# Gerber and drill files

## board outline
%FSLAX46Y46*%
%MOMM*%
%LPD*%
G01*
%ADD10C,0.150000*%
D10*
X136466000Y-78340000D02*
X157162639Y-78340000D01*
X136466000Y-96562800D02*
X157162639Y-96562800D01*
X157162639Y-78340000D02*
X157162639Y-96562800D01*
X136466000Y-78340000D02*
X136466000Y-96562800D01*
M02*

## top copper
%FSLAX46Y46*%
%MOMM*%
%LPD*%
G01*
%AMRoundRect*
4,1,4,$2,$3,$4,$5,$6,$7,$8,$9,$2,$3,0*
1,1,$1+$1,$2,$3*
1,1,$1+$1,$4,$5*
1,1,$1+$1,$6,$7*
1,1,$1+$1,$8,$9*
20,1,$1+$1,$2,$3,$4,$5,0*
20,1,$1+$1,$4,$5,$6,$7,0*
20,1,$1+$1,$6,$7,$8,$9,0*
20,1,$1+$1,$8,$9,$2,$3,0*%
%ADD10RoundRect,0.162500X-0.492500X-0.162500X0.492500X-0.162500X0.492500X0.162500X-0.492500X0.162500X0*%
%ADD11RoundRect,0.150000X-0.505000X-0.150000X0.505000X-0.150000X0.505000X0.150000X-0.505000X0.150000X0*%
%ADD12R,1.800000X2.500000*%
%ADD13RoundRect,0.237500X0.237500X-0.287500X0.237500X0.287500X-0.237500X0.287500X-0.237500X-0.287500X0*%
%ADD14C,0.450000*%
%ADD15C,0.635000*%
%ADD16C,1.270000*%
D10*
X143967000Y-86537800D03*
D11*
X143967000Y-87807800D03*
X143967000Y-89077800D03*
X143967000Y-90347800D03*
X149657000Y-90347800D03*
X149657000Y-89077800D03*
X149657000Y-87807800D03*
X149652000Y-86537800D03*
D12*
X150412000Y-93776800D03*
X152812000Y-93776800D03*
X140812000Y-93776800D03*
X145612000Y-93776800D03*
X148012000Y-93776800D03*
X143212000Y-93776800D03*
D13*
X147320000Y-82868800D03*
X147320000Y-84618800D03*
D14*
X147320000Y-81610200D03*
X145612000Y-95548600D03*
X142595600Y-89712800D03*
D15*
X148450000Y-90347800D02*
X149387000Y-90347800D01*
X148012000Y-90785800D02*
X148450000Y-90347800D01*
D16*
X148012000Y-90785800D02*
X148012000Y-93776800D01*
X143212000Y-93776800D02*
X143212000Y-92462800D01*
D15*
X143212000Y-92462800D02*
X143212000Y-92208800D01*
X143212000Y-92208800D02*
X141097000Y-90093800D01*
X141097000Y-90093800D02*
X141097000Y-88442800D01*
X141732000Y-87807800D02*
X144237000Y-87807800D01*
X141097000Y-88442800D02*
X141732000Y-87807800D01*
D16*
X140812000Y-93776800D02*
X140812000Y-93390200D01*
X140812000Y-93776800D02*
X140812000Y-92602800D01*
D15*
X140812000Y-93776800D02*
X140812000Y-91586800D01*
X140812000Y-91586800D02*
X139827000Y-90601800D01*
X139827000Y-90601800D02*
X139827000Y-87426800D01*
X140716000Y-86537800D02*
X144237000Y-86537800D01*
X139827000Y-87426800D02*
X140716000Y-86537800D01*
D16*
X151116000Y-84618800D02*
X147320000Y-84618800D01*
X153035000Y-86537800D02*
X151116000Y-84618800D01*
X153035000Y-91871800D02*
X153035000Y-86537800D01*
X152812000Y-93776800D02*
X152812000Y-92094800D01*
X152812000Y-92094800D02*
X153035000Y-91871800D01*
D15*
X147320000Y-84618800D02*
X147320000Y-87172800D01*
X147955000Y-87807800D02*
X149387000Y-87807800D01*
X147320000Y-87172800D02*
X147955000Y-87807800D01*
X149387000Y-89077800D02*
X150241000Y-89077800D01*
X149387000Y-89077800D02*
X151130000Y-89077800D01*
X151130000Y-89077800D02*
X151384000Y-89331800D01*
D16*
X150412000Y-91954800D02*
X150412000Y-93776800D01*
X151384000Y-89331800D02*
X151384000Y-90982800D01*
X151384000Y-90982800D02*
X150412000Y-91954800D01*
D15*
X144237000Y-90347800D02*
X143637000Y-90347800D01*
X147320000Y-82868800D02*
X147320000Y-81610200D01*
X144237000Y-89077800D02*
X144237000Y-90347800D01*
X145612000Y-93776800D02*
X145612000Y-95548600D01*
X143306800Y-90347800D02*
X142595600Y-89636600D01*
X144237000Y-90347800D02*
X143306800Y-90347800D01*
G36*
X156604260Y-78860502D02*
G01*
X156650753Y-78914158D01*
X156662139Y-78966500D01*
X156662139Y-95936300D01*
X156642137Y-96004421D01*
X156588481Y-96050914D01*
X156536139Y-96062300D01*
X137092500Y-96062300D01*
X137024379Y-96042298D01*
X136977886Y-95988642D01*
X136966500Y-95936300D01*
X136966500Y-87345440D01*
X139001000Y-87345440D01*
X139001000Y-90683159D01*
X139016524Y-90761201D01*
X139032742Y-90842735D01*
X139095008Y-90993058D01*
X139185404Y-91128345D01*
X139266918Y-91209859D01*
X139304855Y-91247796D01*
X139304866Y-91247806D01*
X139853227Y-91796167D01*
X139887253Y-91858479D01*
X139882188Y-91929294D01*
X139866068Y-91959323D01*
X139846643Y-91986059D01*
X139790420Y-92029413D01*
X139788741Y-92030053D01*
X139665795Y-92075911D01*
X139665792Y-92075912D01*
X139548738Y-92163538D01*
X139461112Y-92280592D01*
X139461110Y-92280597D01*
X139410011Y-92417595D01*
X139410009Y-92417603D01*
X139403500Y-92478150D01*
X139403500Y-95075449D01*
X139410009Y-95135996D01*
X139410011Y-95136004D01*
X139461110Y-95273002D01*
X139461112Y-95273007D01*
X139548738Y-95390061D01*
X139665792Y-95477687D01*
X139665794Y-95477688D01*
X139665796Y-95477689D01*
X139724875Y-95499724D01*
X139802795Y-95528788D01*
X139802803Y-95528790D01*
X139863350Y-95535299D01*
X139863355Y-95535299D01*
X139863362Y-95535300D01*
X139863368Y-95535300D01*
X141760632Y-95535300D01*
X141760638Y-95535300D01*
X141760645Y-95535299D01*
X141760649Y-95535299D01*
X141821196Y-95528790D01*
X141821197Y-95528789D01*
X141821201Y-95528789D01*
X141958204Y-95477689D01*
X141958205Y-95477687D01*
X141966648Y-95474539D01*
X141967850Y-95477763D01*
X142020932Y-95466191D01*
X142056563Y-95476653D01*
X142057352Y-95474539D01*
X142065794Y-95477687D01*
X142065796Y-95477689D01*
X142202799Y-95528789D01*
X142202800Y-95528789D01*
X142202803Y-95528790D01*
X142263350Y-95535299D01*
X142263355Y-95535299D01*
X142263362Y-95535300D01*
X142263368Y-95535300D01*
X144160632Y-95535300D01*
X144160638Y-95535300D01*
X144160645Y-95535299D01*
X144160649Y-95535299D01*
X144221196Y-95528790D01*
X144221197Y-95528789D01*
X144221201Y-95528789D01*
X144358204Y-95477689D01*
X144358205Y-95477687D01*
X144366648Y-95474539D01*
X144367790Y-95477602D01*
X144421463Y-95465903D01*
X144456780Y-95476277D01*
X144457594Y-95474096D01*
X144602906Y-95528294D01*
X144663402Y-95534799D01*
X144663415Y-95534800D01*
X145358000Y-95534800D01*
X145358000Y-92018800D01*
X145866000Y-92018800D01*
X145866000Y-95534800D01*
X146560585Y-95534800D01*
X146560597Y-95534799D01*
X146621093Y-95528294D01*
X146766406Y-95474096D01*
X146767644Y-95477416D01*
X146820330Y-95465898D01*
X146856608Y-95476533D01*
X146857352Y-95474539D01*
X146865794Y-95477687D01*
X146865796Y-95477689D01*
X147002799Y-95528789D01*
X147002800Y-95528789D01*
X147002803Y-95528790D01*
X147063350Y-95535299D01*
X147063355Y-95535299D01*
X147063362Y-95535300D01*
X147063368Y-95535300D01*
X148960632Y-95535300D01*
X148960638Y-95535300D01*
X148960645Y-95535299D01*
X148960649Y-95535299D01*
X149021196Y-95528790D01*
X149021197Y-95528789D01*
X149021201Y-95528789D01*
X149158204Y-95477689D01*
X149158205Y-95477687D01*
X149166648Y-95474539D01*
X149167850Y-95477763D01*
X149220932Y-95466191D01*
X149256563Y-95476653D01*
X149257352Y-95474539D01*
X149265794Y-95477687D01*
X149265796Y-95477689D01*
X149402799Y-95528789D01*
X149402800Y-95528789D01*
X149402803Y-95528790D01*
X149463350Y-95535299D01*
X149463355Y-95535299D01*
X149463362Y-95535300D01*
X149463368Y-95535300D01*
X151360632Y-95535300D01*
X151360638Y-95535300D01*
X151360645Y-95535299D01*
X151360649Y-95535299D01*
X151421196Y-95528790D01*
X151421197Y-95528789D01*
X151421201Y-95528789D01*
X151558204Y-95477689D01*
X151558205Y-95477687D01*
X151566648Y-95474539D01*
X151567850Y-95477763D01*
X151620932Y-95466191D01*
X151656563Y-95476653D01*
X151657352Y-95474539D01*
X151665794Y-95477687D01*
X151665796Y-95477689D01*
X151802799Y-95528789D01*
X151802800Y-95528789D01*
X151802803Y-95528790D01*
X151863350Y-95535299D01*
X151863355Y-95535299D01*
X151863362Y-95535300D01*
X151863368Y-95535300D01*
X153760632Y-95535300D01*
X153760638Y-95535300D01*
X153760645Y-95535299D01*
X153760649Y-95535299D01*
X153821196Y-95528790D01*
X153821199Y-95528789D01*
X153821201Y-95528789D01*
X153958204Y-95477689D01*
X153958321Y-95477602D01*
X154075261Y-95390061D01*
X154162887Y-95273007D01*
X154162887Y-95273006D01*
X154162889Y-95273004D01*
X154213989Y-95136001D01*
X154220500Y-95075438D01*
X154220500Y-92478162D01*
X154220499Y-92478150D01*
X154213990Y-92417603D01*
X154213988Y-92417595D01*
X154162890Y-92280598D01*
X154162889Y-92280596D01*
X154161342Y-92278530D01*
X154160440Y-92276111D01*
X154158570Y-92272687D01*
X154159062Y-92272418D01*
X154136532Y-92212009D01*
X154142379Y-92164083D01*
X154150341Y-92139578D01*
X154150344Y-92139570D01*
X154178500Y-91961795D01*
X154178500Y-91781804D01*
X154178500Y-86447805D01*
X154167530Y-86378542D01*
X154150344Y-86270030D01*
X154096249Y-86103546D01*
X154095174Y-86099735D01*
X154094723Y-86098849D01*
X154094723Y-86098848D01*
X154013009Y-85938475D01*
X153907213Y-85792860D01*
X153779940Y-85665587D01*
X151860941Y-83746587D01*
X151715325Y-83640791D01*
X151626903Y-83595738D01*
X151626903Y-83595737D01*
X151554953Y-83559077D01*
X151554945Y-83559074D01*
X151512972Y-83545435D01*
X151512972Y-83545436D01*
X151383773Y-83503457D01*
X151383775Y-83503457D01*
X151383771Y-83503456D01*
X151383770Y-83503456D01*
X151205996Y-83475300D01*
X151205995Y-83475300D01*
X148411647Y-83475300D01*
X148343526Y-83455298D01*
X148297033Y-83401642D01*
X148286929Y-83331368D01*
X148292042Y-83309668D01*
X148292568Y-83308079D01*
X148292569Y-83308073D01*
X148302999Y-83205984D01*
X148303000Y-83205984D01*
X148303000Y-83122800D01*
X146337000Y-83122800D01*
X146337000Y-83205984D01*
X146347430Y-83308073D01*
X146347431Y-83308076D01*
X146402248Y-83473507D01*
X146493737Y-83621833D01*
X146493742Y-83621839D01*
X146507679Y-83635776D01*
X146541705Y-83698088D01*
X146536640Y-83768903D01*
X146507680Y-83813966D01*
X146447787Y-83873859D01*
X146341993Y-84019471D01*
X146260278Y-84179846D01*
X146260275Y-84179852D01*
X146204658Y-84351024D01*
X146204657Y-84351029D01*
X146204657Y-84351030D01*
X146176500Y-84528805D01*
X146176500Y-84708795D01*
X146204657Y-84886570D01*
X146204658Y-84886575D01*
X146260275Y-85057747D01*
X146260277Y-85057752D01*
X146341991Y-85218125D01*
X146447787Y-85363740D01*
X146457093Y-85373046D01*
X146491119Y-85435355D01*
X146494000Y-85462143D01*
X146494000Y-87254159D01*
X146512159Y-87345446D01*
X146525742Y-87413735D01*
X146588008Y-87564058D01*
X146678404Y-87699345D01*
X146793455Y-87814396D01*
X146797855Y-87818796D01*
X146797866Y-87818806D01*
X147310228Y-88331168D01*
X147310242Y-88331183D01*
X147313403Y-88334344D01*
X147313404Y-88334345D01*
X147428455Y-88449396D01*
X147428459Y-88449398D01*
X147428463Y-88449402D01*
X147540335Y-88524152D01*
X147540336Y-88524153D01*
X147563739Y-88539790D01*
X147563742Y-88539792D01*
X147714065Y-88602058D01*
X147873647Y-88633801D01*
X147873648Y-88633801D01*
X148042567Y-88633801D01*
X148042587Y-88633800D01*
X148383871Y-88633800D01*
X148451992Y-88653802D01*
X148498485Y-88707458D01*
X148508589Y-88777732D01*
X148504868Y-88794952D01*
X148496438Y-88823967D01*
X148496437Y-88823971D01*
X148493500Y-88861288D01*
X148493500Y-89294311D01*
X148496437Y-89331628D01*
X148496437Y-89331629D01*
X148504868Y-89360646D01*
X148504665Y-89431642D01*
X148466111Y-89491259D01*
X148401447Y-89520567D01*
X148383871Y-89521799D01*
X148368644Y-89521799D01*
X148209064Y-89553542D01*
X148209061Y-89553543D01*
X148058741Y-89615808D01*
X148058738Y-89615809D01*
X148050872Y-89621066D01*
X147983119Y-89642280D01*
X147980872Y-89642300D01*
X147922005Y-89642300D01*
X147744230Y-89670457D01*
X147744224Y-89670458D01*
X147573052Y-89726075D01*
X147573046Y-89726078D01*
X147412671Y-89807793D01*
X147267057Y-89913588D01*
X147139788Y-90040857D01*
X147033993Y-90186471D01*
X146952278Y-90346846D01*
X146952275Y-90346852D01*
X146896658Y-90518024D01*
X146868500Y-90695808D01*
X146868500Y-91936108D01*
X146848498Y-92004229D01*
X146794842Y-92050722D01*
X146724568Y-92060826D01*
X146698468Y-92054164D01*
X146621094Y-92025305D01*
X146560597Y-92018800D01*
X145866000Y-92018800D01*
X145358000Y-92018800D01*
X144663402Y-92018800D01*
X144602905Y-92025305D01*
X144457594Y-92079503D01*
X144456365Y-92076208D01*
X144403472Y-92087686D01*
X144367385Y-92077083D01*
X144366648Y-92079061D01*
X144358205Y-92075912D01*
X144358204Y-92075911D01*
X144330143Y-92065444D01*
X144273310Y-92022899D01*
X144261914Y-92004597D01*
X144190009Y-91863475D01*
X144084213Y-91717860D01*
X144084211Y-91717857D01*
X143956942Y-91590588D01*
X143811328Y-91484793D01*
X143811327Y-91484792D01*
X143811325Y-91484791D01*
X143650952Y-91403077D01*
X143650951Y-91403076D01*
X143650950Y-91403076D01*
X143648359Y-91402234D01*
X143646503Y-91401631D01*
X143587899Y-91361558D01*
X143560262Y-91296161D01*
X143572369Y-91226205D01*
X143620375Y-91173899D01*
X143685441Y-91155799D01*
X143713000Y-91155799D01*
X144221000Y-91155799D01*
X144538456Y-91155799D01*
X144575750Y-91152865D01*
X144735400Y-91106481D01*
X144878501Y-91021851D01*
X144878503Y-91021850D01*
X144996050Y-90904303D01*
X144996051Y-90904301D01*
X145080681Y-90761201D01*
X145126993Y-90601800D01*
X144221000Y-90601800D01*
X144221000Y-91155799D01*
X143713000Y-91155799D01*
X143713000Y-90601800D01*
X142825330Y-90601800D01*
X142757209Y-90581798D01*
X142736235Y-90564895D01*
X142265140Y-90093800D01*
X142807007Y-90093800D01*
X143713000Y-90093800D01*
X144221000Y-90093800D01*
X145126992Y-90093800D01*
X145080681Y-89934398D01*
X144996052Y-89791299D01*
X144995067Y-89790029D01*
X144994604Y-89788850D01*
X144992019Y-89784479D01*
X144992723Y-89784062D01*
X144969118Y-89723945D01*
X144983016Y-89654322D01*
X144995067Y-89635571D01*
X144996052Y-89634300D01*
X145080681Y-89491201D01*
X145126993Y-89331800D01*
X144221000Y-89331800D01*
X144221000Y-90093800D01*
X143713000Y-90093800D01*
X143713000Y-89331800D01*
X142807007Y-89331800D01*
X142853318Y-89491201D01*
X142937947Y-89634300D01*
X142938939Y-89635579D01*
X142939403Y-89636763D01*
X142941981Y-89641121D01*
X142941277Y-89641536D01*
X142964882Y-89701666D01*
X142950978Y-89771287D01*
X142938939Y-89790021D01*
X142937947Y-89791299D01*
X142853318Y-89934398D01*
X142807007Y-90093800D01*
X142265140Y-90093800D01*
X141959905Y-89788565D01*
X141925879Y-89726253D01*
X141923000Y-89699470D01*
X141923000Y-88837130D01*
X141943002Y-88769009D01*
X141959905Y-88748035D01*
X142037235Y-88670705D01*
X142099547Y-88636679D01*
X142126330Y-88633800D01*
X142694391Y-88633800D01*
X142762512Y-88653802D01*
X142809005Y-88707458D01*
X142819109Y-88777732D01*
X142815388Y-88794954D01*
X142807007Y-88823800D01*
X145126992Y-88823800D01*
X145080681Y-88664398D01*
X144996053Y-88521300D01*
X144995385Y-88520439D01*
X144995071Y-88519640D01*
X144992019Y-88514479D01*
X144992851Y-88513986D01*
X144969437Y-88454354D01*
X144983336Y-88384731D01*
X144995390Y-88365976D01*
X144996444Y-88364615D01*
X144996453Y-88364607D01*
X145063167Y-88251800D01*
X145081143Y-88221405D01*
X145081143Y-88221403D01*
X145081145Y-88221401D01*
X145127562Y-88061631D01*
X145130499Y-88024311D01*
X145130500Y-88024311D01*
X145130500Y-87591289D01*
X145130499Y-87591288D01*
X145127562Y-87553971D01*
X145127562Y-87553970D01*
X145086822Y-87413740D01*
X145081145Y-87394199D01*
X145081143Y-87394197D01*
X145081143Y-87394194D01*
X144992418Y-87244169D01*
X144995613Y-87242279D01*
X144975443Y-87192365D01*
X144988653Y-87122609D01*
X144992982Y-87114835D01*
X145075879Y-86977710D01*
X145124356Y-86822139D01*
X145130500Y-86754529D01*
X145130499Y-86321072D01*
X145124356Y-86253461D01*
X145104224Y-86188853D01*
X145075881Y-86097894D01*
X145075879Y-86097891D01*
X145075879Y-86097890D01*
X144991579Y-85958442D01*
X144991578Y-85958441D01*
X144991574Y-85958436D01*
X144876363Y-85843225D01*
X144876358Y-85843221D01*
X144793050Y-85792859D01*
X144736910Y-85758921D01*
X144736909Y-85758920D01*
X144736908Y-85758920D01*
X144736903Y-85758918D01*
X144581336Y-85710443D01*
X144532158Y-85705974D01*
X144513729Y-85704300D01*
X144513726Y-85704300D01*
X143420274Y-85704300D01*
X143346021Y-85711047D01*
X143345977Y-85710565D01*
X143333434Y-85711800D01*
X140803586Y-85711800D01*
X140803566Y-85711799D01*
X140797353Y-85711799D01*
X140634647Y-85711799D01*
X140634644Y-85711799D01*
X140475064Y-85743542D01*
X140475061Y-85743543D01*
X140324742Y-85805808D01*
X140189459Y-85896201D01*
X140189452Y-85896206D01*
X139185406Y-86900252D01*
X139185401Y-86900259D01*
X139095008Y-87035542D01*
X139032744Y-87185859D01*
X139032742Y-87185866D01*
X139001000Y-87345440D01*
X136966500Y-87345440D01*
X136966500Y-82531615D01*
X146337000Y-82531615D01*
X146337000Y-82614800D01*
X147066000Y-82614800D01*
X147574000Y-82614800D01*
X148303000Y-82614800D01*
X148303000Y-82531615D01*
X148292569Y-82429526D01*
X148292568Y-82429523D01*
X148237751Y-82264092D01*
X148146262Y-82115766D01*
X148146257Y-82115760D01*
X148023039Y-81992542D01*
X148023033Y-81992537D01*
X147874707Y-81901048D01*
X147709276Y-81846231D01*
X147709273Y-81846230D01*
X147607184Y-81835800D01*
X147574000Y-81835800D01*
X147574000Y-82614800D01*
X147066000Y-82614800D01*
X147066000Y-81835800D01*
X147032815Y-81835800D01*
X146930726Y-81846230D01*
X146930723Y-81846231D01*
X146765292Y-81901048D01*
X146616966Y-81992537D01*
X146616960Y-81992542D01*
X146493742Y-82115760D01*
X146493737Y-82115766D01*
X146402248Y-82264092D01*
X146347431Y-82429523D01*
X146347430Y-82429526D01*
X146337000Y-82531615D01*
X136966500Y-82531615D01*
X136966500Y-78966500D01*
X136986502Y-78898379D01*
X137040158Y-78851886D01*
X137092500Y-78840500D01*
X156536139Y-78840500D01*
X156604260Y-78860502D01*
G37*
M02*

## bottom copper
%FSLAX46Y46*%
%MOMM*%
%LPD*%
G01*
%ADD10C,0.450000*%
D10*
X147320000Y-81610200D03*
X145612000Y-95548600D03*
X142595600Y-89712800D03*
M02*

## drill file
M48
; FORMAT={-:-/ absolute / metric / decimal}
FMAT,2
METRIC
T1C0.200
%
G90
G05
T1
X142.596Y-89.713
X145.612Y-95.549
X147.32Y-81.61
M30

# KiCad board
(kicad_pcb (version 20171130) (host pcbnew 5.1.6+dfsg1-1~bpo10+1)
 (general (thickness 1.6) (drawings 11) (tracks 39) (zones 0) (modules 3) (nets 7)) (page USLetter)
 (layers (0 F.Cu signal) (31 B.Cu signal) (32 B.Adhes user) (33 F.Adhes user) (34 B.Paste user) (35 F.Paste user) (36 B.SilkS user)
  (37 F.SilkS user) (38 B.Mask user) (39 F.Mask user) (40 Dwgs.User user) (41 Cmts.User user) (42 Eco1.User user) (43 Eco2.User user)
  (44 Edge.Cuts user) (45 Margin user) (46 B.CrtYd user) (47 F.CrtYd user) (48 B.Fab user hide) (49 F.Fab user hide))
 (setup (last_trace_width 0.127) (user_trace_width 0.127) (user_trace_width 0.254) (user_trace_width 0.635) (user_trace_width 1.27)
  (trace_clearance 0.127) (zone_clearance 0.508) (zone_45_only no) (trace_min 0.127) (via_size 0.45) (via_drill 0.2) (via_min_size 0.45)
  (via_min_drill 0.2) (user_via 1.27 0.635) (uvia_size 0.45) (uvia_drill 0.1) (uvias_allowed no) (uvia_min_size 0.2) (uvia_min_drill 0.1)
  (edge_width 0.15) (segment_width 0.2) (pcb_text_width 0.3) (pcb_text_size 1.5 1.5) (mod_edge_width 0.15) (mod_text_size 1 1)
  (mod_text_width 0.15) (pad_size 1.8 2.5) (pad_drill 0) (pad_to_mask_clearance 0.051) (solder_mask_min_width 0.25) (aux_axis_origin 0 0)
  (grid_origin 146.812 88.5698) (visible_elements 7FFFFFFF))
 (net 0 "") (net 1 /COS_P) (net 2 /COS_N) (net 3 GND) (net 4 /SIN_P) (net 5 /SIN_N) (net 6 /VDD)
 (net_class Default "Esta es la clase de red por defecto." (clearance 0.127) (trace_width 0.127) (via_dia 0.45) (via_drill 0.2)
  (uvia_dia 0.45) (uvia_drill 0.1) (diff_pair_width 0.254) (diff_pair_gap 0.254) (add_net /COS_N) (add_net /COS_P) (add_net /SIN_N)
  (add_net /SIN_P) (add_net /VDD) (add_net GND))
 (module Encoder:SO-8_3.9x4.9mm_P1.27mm (layer F.Cu) (at 146.812 88.4428)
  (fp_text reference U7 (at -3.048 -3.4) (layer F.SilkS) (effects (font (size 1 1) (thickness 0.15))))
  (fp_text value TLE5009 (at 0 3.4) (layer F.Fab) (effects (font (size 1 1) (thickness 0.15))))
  (pad 1 smd roundrect (at -2.845 -1.905) (size 1.31 0.65) (layers F.Cu F.Paste F.Mask) (roundrect_rratio 0.25) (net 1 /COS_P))
  (pad 2 smd roundrect (at -2.845 -0.635) (size 1.31 0.6) (layers F.Cu F.Paste F.Mask) (roundrect_rratio 0.25) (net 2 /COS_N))
  (pad 3 smd roundrect (at -2.845 0.635) (size 1.31 0.6) (layers F.Cu F.Paste F.Mask) (roundrect_rratio 0.25) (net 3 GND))
  (pad 4 smd roundrect (at -2.845 1.905) (size 1.31 0.6) (layers F.Cu F.Paste F.Mask) (roundrect_rratio 0.25) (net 3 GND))
  (pad 5 smd roundrect (at 2.845 1.905) (size 1.31 0.6) (layers F.Cu F.Paste F.Mask) (roundrect_rratio 0.25) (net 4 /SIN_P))
  (pad 6 smd roundrect (at 2.845 0.635) (size 1.31 0.6) (layers F.Cu F.Paste F.Mask) (roundrect_rratio 0.25) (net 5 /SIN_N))
  (pad 7 smd roundrect (at 2.845 -0.635) (size 1.31 0.6) (layers F.Cu F.Paste F.Mask) (roundrect_rratio 0.25) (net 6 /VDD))
  (pad 8 smd roundrect (at 2.84 -1.905) (size 1.31 0.6) (layers F.Cu F.Paste F.Mask) (roundrect_rratio 0.25)))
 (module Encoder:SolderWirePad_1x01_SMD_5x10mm (layer F.Cu) (at 146.812 93.7768)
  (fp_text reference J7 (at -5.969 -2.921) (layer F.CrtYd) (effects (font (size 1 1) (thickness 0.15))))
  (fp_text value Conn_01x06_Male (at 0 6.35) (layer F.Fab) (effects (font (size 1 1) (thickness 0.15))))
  (pad 5 smd rect (at 3.6 0) (size 1.8 2.5) (layers F.Cu F.Paste F.Mask) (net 5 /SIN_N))
  (pad 6 smd rect (at 6 0) (size 1.8 2.5) (layers F.Cu F.Paste F.Mask) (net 6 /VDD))
  (pad 1 smd rect (at -6 0) (size 1.8 2.5) (layers F.Cu F.Paste F.Mask) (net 1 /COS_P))
  (pad 3 smd rect (at -1.2 0) (size 1.8 2.5) (layers F.Cu F.Paste F.Mask) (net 3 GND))
  (pad 4 smd rect (at 1.2 0) (size 1.8 2.5) (layers F.Cu F.Paste F.Mask) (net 4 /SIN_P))
  (pad 2 smd rect (at -3.6 0) (size 1.8 2.5) (layers F.Cu F.Paste F.Mask) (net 2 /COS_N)))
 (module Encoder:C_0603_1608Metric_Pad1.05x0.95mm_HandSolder (layer F.Cu) (at 147.32 83.7438 90)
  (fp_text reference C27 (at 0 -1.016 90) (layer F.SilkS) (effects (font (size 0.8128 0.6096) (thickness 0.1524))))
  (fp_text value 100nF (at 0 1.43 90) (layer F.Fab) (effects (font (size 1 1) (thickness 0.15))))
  (pad 2 smd roundrect (at 0.875 0 90) (size 1.05 0.95) (layers F.Cu F.Paste F.Mask) (roundrect_rratio 0.25) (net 3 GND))
  (pad 1 smd roundrect (at -0.875 0 90) (size 1.05 0.95) (layers F.Cu F.Paste F.Mask) (roundrect_rratio 0.25) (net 6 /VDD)))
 (gr_line (start 136.466 78.34) (end 157.162639 78.34) (layer Edge.Cuts) (width 0.15))
 (gr_line (start 136.466 96.5628) (end 157.162639 96.5628) (layer Edge.Cuts) (width 0.15))
 (gr_line (start 157.162639 78.34) (end 157.162639 96.5628) (layer Edge.Cuts) (width 0.15))
 (gr_line (start 136.466 78.34) (end 136.466 96.5628) (layer Edge.Cuts) (width 0.15))
 (segment (start 148.45 90.3478) (end 149.387 90.3478) (width 0.635) (layer F.Cu) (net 4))
 (segment (start 148.012 90.7858) (end 148.45 90.3478) (width 0.635) (layer F.Cu) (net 4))
 (segment (start 148.012 90.7858) (end 148.012 93.7768) (width 1.27) (layer F.Cu) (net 4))
 (segment (start 143.212 93.7768) (end 143.212 92.4628) (width 1.27) (layer F.Cu) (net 2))
 (segment (start 143.212 92.4628) (end 143.212 92.2088) (width 0.635) (layer F.Cu) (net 2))
 (segment (start 143.212 92.2088) (end 141.097 90.0938) (width 0.635) (layer F.Cu) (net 2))
 (segment (start 141.097 90.0938) (end 141.097 88.4428) (width 0.635) (layer F.Cu) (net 2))
 (segment (start 141.732 87.8078) (end 144.237 87.8078) (width 0.635) (layer F.Cu) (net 2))
 (segment (start 141.097 88.4428) (end 141.732 87.8078) (width 0.635) (layer F.Cu) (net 2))
 (segment (start 140.812 93.7768) (end 140.812 93.3902) (width 1.27) (layer F.Cu) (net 1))
 (segment (start 140.812 93.7768) (end 140.812 92.6028) (width 1.27) (layer F.Cu) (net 1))
 (segment (start 140.812 93.7768) (end 140.812 91.5868) (width 0.635) (layer F.Cu) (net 1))
 (segment (start 140.812 91.5868) (end 139.827 90.6018) (width 0.635) (layer F.Cu) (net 1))
 (segment (start 139.827 90.6018) (end 139.827 87.4268) (width 0.635) (layer F.Cu) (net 1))
 (segment (start 140.716 86.5378) (end 144.237 86.5378) (width 0.635) (layer F.Cu) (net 1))
 (segment (start 139.827 87.4268) (end 140.716 86.5378) (width 0.635) (layer F.Cu) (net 1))
 (segment (start 151.116 84.6188) (end 147.32 84.6188) (width 1.27) (layer F.Cu) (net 6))
 (segment (start 153.035 86.5378) (end 151.116 84.6188) (width 1.27) (layer F.Cu) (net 6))
 (segment (start 153.035 91.8718) (end 153.035 86.5378) (width 1.27) (layer F.Cu) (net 6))
 (segment (start 152.812 93.7768) (end 152.812 92.0948) (width 1.27) (layer F.Cu) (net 6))
 (segment (start 152.812 92.0948) (end 153.035 91.8718) (width 1.27) (layer F.Cu) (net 6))
 (segment (start 147.32 84.6188) (end 147.32 87.1728) (width 0.635) (layer F.Cu) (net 6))
 (segment (start 147.955 87.8078) (end 149.387 87.8078) (width 0.635) (layer F.Cu) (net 6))
 (segment (start 147.32 87.1728) (end 147.955 87.8078) (width 0.635) (layer F.Cu) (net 6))
 (segment (start 149.387 89.0778) (end 150.241 89.0778) (width 0.635) (layer F.Cu) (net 5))
 (segment (start 149.387 89.0778) (end 151.13 89.0778) (width 0.635) (layer F.Cu) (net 5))
 (segment (start 151.13 89.0778) (end 151.384 89.3318) (width 0.635) (layer F.Cu) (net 5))
 (segment (start 150.412 91.9548) (end 150.412 93.7768) (width 1.27) (layer F.Cu) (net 5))
 (segment (start 151.384 89.3318) (end 151.384 90.9828) (width 1.27) (layer F.Cu) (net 5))
 (segment (start 151.384 90.9828) (end 150.412 91.9548) (width 1.27) (layer F.Cu) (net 5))
 (segment (start 144.237 90.3478) (end 143.637 90.3478) (width 0.635) (layer F.Cu) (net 3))
 (segment (start 147.32 82.8688) (end 147.32 81.6102) (width 0.635) (layer F.Cu) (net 3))
 (via (at 147.32 81.6102) (size 0.45) (drill 0.2) (layers F.Cu B.Cu) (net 3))
 (segment (start 144.237 89.0778) (end 144.237 90.3478) (width 0.635) (layer F.Cu) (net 3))
 (segment (start 145.612 93.7768) (end 145.612 95.5486) (width 0.635) (layer F.Cu) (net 3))
 (via (at 145.612 95.5486) (size 0.45) (drill 0.2) (layers F.Cu B.Cu) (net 3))
 (via (at 142.5956 89.7128) (size 0.45) (drill 0.2) (layers F.Cu B.Cu) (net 3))
 (segment (start 143.3068 90.3478) (end 142.5956 89.6366) (width 0.635) (layer F.Cu) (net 3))
 (segment (start 144.237 90.3478) (end 143.3068 90.3478) (width 0.635) (layer F.Cu) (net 3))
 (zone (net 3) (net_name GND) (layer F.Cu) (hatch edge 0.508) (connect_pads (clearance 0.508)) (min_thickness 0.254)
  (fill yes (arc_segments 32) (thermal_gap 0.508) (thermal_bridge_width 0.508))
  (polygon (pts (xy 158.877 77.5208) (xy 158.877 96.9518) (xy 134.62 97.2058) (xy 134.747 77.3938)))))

